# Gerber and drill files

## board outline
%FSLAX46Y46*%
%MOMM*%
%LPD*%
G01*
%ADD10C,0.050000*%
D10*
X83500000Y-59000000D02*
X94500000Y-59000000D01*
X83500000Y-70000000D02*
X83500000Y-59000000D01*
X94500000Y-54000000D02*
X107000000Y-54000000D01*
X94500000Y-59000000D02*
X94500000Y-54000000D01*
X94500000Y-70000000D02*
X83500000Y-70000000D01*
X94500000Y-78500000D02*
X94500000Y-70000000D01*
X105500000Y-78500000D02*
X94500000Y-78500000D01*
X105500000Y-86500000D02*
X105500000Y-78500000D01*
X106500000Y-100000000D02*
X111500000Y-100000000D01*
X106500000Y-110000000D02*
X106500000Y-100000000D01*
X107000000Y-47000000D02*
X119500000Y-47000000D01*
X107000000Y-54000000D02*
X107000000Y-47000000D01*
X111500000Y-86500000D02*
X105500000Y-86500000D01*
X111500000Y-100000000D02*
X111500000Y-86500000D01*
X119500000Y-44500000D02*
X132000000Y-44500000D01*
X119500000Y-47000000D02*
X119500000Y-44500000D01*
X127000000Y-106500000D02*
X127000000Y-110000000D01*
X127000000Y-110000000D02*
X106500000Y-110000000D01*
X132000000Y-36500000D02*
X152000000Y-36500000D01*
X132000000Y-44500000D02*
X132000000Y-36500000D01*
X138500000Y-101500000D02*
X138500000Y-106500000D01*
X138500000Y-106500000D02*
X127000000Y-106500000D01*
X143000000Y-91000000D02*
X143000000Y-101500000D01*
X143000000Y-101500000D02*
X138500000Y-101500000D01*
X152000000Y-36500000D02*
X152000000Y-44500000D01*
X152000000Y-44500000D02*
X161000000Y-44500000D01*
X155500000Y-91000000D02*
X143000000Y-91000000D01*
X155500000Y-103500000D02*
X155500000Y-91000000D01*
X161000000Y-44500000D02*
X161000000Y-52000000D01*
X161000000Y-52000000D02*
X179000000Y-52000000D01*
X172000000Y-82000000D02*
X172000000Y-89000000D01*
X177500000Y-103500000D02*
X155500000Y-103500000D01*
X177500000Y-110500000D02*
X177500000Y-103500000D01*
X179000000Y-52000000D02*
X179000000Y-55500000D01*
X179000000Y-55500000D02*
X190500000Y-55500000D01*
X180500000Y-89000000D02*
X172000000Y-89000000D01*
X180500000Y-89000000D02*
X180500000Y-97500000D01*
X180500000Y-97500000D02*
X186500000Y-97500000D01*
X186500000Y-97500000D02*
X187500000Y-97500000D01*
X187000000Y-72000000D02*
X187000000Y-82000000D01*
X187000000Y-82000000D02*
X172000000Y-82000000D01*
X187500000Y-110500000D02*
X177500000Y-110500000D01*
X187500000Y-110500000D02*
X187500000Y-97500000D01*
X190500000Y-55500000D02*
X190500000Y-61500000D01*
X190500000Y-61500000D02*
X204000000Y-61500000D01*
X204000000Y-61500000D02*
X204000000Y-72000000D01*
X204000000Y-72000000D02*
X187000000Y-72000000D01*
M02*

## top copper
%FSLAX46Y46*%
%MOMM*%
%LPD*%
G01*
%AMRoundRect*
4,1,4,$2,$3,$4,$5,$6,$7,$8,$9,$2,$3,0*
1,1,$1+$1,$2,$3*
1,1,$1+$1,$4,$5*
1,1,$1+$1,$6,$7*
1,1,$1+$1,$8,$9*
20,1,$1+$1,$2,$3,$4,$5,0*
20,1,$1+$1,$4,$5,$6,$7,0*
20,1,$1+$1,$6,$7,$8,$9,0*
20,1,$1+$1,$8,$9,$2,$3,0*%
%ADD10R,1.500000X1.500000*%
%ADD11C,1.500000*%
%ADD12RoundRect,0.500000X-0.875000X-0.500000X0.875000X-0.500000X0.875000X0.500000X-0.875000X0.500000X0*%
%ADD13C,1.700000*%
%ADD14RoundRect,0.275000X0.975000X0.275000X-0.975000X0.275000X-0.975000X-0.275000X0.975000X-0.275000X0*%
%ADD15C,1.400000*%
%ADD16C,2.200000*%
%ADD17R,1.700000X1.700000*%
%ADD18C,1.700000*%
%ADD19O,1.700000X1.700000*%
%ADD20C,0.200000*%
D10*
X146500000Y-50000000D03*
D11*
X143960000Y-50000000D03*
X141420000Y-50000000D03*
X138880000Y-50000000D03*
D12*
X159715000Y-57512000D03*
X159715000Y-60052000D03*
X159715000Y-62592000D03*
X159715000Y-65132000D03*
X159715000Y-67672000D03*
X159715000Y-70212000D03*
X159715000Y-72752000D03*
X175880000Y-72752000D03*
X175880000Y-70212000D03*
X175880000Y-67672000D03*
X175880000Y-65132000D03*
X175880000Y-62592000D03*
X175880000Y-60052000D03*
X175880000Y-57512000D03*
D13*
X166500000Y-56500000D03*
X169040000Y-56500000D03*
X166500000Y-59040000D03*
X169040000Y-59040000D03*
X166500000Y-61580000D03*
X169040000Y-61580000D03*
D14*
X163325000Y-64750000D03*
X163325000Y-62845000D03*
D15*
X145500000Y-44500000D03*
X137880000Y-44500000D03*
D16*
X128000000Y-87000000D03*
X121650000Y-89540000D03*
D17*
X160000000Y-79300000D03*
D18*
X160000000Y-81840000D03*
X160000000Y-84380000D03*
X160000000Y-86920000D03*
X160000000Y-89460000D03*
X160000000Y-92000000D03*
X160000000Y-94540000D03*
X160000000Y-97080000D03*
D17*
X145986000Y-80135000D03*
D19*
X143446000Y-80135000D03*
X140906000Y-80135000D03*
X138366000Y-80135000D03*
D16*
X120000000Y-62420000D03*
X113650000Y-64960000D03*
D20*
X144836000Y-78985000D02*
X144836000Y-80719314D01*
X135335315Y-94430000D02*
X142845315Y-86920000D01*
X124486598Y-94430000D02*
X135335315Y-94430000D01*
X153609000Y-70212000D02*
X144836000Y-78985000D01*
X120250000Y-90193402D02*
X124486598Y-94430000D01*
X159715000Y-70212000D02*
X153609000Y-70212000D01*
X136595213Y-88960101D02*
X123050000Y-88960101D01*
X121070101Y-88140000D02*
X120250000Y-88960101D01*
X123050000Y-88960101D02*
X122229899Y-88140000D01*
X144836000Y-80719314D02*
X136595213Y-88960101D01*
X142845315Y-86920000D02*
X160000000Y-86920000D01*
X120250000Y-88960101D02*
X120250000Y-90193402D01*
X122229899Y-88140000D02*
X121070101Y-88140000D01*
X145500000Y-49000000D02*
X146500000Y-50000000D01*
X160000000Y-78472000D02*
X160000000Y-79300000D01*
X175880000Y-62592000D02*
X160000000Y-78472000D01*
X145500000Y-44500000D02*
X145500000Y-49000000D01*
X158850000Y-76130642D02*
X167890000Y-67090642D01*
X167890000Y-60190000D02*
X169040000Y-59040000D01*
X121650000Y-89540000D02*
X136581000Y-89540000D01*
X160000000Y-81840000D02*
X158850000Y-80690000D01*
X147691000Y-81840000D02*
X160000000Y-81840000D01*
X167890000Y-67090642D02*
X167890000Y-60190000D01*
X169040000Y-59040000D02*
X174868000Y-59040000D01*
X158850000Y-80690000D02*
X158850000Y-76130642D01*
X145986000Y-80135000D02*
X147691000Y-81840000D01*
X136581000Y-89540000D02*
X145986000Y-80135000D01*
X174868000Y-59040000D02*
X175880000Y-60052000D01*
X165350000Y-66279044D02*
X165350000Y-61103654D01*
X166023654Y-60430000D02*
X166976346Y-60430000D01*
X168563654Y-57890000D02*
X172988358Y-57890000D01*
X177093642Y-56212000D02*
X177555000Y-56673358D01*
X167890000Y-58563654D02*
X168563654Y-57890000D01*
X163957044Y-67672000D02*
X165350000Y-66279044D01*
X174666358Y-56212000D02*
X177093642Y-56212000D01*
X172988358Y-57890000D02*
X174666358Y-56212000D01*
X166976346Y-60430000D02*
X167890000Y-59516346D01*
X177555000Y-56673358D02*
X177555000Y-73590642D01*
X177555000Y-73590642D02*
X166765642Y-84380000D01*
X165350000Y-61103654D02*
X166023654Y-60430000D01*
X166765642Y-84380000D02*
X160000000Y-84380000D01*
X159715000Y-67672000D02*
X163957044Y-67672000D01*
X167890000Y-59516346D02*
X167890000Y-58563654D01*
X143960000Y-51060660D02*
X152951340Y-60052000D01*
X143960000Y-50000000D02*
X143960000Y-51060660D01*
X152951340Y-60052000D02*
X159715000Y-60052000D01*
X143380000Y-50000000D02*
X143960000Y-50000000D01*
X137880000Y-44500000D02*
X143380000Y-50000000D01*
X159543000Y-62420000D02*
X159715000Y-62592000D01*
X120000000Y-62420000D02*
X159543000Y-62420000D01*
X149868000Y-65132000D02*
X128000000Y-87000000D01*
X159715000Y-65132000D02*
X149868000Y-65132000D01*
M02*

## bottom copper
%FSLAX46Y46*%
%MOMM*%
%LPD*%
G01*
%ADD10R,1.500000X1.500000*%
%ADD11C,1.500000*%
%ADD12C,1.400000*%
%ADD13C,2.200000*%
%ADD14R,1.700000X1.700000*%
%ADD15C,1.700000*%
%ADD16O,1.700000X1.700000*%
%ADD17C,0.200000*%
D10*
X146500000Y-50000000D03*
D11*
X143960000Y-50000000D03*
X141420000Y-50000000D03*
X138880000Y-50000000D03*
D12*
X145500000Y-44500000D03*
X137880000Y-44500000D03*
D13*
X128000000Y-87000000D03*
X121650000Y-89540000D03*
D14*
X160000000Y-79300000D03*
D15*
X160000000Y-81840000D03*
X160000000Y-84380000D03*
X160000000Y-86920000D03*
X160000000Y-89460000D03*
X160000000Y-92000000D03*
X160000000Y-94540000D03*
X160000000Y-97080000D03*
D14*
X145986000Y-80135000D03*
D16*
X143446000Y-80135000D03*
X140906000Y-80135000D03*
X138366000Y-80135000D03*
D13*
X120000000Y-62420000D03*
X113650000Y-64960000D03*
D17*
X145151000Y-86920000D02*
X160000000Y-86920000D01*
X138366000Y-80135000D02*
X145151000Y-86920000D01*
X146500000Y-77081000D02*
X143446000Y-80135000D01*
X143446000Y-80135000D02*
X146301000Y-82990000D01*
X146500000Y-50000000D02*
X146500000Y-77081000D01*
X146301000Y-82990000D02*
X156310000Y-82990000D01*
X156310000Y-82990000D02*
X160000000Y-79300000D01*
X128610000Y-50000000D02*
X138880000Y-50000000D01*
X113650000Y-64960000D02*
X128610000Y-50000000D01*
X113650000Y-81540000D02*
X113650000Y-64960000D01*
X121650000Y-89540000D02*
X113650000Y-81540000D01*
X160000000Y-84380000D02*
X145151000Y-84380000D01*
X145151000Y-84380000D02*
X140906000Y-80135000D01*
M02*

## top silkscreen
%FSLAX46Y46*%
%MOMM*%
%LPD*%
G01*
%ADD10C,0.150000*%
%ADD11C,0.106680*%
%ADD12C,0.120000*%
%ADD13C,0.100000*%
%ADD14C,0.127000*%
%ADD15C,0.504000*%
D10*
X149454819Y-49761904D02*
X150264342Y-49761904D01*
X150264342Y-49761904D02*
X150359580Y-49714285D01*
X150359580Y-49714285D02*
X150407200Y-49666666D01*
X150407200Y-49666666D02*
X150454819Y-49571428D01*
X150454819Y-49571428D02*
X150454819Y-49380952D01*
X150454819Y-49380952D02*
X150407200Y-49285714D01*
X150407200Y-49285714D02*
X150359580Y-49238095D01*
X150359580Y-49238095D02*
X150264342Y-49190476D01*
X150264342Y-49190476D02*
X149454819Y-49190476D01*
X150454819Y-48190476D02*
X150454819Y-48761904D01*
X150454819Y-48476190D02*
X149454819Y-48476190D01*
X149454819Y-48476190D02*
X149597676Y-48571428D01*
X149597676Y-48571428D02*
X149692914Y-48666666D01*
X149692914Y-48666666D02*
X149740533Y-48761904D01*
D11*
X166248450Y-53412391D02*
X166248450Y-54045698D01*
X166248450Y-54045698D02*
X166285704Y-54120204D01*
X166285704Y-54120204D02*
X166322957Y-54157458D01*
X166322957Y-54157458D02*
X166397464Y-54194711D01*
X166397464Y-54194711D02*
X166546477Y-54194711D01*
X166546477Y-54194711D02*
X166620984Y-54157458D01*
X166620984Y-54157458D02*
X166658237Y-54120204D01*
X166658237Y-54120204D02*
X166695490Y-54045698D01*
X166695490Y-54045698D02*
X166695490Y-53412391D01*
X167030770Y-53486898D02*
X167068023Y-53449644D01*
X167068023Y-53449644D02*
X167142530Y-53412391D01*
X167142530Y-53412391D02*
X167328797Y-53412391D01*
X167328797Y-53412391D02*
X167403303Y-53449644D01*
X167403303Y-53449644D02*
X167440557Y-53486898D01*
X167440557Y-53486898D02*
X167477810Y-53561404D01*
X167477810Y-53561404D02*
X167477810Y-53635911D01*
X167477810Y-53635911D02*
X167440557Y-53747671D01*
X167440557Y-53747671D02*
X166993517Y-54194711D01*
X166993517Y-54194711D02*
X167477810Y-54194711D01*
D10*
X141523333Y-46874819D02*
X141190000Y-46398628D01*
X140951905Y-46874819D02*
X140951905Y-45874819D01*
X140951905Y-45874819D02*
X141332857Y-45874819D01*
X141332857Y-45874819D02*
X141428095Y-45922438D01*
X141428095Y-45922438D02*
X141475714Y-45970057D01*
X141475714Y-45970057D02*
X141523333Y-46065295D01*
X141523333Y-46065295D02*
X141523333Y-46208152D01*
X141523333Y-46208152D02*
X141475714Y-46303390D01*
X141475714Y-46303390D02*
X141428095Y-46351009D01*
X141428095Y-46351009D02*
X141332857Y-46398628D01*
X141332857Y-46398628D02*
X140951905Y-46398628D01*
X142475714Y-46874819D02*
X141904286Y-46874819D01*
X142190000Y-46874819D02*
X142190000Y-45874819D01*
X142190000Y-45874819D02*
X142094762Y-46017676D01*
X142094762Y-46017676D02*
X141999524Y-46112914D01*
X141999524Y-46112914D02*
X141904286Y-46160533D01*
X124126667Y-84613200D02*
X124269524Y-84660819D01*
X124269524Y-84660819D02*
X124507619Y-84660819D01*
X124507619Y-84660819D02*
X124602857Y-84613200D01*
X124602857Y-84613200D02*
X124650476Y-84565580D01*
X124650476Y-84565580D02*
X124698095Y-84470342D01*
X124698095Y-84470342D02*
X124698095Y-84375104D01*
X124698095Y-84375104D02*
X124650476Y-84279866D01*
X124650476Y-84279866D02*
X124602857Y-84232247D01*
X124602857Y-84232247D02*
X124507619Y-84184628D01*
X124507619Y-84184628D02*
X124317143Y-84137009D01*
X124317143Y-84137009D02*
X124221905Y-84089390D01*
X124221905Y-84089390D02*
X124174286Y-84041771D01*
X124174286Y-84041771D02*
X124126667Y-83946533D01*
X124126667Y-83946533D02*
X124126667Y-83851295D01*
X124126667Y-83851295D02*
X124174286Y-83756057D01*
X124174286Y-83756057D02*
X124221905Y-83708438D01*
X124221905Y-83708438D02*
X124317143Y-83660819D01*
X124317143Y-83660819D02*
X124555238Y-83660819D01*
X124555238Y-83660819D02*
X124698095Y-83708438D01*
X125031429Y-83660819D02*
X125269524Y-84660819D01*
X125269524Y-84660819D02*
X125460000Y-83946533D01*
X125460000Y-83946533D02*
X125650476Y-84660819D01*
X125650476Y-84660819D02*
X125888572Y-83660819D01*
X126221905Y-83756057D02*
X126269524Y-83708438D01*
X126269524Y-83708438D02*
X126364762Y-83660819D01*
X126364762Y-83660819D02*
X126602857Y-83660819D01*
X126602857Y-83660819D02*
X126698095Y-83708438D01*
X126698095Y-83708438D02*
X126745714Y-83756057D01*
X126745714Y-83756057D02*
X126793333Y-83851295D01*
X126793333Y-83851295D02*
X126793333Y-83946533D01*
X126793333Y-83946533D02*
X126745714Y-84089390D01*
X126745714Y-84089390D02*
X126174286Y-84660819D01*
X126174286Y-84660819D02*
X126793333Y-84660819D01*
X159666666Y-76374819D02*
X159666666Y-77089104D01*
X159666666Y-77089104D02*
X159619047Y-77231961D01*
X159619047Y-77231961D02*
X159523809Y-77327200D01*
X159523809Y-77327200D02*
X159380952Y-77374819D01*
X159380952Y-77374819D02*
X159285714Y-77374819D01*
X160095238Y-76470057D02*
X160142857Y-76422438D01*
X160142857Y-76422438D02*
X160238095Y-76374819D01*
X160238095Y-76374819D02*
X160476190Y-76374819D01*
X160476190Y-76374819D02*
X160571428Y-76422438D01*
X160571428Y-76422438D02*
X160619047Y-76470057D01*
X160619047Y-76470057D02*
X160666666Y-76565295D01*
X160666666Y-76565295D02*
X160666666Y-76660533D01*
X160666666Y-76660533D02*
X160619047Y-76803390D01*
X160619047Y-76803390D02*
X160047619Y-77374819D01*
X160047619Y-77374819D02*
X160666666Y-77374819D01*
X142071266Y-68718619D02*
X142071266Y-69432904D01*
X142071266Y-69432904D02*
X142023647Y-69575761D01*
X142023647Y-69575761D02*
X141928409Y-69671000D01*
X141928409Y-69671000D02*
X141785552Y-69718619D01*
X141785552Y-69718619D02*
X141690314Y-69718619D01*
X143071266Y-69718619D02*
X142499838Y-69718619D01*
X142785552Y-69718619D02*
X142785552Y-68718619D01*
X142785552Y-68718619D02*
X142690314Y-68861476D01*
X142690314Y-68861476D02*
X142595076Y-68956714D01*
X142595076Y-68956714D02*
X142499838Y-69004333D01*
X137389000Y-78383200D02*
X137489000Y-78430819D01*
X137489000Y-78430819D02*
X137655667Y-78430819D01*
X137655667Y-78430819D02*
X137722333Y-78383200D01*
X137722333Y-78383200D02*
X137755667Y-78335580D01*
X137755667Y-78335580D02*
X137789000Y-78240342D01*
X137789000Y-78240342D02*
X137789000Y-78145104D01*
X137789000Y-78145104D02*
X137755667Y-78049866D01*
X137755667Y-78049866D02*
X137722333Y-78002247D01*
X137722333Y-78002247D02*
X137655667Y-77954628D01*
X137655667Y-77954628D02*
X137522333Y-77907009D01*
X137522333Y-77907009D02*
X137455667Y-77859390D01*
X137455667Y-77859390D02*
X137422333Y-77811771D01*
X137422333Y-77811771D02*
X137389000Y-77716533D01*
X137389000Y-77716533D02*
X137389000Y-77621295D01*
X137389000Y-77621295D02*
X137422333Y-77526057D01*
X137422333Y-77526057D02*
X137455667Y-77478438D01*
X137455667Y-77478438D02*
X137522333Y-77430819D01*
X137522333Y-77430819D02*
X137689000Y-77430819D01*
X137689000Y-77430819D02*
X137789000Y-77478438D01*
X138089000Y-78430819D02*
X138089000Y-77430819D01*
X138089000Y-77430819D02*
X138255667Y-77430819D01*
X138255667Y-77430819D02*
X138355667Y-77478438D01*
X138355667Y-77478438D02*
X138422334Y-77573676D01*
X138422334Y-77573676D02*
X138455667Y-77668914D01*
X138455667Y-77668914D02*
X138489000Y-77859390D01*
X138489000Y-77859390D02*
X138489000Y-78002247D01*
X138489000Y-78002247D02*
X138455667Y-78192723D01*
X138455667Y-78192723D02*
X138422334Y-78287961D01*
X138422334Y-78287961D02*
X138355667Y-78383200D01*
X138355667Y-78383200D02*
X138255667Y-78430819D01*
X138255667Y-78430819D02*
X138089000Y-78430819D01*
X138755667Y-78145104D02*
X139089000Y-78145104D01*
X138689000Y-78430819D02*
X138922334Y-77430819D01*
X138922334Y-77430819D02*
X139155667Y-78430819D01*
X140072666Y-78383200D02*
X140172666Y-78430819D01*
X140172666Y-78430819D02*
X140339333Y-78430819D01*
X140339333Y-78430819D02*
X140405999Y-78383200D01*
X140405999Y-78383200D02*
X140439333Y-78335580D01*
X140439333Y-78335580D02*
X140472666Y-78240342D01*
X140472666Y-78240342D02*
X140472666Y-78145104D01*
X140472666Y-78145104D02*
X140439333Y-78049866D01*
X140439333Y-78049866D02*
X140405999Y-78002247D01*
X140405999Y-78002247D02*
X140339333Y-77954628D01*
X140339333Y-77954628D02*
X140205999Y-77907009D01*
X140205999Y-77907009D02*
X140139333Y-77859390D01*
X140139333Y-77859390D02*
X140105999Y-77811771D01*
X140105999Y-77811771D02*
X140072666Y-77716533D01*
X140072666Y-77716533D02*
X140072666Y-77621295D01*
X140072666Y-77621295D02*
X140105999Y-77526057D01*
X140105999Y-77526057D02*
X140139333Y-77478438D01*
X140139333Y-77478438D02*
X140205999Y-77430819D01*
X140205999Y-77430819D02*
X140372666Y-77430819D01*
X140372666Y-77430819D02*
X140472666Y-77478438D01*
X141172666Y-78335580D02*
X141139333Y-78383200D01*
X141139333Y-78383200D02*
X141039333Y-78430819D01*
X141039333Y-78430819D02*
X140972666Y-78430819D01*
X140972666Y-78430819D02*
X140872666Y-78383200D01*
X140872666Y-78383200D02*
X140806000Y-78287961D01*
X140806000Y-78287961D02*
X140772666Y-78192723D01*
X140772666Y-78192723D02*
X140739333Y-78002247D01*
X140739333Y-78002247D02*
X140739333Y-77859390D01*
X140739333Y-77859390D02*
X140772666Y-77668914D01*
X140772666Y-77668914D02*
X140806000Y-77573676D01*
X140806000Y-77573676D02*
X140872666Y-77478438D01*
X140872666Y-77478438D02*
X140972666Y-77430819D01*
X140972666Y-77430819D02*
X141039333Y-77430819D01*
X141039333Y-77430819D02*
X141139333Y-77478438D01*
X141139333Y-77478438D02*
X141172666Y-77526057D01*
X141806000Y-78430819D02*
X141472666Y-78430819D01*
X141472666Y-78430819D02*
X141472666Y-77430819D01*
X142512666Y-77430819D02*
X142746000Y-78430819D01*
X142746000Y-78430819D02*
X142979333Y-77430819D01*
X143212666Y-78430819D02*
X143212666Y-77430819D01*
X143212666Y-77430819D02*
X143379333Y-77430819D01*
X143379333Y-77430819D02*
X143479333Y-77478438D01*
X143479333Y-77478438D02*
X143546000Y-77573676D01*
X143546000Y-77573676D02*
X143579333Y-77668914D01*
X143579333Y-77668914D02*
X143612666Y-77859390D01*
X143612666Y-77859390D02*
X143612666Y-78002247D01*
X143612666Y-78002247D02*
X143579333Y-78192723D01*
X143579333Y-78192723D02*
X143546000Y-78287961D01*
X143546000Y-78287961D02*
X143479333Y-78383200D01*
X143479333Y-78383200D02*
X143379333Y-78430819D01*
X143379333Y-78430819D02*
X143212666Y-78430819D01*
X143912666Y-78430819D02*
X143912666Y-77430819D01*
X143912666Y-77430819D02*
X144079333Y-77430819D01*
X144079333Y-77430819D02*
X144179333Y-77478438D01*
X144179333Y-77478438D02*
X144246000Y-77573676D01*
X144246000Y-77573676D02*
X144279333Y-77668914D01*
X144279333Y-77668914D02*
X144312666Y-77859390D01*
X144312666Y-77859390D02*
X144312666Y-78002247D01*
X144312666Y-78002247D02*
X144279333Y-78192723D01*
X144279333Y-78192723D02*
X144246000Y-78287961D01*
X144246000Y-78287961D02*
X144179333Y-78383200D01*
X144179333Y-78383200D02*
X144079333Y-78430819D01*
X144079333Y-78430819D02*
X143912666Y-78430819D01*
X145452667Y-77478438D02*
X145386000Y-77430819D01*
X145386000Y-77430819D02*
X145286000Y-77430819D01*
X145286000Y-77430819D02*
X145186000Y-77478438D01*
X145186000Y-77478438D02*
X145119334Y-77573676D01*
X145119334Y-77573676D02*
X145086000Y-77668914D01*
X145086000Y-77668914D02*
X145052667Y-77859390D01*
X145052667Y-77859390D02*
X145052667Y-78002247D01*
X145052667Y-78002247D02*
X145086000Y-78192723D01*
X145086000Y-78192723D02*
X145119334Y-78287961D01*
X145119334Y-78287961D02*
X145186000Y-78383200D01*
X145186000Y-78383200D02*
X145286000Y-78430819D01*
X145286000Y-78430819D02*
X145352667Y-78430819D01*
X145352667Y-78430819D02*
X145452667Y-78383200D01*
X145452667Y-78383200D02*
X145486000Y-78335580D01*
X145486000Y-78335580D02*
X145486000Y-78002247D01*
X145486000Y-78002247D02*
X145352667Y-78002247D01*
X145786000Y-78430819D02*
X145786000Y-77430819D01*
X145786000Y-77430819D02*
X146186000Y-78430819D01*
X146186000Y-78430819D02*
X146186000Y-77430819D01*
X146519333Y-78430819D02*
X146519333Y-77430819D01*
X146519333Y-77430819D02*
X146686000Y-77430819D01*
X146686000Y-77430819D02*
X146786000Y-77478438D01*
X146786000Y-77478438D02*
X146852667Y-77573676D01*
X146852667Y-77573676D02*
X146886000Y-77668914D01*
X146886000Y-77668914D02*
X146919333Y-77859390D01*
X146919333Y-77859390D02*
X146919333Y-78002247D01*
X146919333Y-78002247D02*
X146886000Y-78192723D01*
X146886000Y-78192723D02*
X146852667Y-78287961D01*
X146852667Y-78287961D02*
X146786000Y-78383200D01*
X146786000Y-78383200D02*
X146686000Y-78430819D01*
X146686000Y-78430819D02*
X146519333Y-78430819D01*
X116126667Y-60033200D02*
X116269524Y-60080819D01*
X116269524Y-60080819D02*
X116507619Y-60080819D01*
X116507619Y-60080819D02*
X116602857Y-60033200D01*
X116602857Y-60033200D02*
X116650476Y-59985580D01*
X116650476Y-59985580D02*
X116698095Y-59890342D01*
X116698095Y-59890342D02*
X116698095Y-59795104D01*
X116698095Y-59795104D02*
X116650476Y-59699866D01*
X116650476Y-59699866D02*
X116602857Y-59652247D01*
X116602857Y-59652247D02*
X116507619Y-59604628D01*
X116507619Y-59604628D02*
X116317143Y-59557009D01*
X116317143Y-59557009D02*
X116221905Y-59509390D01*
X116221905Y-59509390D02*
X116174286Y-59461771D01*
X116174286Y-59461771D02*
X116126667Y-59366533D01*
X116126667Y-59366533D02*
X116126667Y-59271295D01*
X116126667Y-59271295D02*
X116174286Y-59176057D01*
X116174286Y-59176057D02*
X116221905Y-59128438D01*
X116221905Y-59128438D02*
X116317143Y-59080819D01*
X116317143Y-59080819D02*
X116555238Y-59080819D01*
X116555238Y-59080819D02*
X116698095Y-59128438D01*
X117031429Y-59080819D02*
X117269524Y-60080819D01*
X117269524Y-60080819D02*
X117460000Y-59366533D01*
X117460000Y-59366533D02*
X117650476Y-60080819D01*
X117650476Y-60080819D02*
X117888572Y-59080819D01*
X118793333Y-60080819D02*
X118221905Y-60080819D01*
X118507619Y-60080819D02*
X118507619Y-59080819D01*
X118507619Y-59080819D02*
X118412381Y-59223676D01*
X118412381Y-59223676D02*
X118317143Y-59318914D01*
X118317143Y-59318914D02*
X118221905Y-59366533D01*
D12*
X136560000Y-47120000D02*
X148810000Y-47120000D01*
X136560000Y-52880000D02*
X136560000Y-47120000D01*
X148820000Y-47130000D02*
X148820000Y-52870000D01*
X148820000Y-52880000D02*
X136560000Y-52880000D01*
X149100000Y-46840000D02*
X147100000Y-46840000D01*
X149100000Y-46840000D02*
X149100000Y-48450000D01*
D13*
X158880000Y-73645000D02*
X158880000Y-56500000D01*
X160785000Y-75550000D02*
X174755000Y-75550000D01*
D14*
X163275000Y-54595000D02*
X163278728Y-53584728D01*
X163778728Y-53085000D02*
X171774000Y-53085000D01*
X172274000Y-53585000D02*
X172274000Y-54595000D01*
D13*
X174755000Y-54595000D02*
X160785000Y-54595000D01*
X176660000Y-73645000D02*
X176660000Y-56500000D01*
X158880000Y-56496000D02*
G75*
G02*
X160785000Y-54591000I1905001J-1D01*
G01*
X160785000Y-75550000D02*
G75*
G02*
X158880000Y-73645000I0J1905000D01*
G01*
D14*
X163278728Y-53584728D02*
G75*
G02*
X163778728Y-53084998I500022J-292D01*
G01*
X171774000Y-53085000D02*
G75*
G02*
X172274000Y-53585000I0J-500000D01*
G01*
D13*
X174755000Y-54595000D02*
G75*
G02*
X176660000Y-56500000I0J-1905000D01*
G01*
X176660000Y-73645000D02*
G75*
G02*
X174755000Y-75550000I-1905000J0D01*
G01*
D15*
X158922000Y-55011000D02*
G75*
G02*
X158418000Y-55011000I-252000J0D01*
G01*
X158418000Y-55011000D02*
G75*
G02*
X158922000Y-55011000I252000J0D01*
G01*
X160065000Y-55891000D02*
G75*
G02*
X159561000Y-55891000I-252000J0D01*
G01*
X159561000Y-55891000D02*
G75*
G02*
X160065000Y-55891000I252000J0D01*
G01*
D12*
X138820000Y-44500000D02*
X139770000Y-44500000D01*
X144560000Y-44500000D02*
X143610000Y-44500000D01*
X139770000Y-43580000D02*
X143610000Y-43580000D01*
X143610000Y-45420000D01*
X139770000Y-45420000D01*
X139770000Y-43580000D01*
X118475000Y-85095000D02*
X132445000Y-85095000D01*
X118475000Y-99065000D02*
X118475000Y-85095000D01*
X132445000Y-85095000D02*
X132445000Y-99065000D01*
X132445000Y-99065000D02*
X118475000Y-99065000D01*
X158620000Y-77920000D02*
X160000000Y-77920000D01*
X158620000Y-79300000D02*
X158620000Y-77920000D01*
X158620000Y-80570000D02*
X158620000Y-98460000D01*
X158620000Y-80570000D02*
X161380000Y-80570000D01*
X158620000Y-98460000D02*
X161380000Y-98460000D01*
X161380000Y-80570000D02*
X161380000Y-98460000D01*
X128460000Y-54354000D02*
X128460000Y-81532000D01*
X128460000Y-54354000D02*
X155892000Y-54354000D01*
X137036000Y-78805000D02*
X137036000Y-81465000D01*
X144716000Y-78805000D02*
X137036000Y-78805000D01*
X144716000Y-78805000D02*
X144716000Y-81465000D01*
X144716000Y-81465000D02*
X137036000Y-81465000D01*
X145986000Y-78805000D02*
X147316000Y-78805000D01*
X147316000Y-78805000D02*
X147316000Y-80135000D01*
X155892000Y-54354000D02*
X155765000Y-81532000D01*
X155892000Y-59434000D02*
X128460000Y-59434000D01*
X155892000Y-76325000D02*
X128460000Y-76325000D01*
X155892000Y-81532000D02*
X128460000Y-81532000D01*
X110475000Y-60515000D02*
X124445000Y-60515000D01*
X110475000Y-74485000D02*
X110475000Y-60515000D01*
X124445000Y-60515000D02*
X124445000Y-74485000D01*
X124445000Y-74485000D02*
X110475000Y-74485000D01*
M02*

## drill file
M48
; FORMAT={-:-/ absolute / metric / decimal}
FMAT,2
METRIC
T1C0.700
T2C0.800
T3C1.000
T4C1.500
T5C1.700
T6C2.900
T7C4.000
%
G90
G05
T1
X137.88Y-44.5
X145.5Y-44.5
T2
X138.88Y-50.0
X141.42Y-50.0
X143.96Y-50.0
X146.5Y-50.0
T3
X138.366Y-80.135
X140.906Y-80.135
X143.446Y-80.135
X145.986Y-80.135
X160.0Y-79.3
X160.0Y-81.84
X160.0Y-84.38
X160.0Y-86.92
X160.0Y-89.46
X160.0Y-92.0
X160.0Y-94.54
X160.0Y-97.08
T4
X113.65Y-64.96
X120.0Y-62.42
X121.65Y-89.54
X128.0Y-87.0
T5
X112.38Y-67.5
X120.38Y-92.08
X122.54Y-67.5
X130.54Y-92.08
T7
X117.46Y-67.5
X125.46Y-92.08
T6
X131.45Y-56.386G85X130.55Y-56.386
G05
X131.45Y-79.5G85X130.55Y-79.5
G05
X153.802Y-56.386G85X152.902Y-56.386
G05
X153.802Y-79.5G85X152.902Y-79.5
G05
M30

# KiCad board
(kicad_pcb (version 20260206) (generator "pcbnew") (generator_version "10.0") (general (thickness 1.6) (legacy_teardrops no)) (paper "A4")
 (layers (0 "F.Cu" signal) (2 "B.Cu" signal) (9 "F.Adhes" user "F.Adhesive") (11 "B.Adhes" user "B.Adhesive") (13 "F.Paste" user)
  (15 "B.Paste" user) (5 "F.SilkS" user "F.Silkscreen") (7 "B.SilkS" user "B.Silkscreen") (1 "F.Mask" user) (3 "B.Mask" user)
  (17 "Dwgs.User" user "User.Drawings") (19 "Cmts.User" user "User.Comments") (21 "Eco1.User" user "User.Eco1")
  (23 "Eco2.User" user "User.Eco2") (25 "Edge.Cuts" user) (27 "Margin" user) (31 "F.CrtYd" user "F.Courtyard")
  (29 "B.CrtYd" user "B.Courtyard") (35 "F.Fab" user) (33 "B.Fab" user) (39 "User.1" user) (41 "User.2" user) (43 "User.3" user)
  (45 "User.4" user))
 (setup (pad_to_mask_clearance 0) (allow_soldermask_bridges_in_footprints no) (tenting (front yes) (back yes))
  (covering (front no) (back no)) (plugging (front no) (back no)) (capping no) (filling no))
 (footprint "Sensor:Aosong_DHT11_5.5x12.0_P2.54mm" (layer "F.Cu") (at 146.5 50 -90)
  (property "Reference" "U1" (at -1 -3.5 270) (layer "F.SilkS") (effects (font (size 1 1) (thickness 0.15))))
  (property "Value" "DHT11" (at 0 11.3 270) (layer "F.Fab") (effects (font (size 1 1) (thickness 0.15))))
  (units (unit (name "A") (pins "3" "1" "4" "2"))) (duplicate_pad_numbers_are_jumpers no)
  (fp_line (start -2.88 9.94) (end -2.88 -2.31) (stroke (width 0.12) (type solid)) (layer "F.SilkS"))
  (fp_line (start 2.88 9.94) (end -2.88 9.94) (stroke (width 0.12) (type solid)) (layer "F.SilkS"))
  (fp_line (start -2.87 -2.32) (end 2.87 -2.32) (stroke (width 0.12) (type solid)) (layer "F.SilkS"))
  (fp_line (start 2.88 -2.32) (end 2.88 9.94) (stroke (width 0.12) (type solid)) (layer "F.SilkS"))
  (fp_line (start -3.16 -2.6) (end -3.16 -0.6) (stroke (width 0.12) (type solid)) (layer "F.SilkS"))
  (fp_line (start -3.16 -2.6) (end -1.55 -2.6) (stroke (width 0.12) (type solid)) (layer "F.SilkS"))
  (pad "1" thru_hole rect (at 0 0 270) (size 1.5 1.5) (drill 0.8) (layers "*.Cu" "*.Mask") (remove_unused_layers no) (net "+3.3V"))
  (pad "2" thru_hole circle (at 0 2.54 270) (size 1.5 1.5) (drill 0.8) (layers "*.Cu" "*.Mask") (remove_unused_layers no)
   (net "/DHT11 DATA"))
  (pad "3" thru_hole circle (at 0 5.08 270) (size 1.5 1.5) (drill 0.8) (layers "*.Cu" "*.Mask") (remove_unused_layers no)
   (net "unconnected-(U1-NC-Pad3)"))
  (pad "4" thru_hole circle (at 0 7.62 270) (size 1.5 1.5) (drill 0.8) (layers "*.Cu" "*.Mask") (remove_unused_layers no) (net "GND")))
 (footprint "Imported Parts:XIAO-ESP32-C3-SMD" (layer "F.Cu") (at 158.88 75.632)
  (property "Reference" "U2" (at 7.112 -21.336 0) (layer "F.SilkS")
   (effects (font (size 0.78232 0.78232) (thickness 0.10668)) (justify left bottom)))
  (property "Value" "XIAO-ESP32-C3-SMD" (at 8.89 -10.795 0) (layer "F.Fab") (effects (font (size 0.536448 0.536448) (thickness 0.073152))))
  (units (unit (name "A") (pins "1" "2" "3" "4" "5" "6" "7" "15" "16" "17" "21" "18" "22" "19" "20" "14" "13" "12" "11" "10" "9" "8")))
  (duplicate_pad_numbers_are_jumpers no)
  (fp_line (start 0 -1.987) (end 0 -19.132) (stroke (width 0.1) (type solid)) (layer "F.SilkS"))
  (fp_line (start 1.905 -0.082) (end 15.875 -0.082) (stroke (width 0.1) (type solid)) (layer "F.SilkS"))
  (fp_line (start 4.395 -21.037) (end 4.398728 -22.047272) (stroke (width 0.127) (type solid)) (layer "F.SilkS"))
  (fp_line (start 4.898728 -22.547) (end 12.894 -22.547) (stroke (width 0.127) (type solid)) (layer "F.SilkS"))
  (fp_line (start 13.394 -22.047) (end 13.394 -21.037) (stroke (width 0.127) (type solid)) (layer "F.SilkS"))
  (fp_line (start 15.875 -21.037) (end 1.905 -21.037) (stroke (width 0.1) (type solid)) (layer "F.SilkS"))
  (fp_line (start 17.78 -1.987) (end 17.78 -19.132) (stroke (width 0.1) (type solid)) (layer "F.SilkS"))
  (fp_arc (start 0 -19.136) (mid 0.557962 -20.483038) (end 1.905 -21.041) (stroke (width 0.1) (type solid)) (layer "F.SilkS"))
  (fp_arc (start 1.905 -0.082) (mid 0.557962 -0.639962) (end 0 -1.987) (stroke (width 0.1) (type solid)) (layer "F.SilkS"))
  (fp_arc (start 4.398728 -22.047272) (mid 4.545272 -22.40064) (end 4.898728 -22.547) (stroke (width 0.127) (type default))
   (layer "F.SilkS"))
  (fp_arc (start 12.894 -22.547) (mid 13.247553 -22.400553) (end 13.394 -22.047) (stroke (width 0.127) (type default)) (layer "F.SilkS"))
  (fp_arc (start 15.875 -21.037) (mid 17.222038 -20.479038) (end 17.78 -19.132) (stroke (width 0.1) (type solid)) (layer "F.SilkS"))
  (fp_arc (start 17.78 -1.987) (mid 17.222038 -0.639962) (end 15.875 -0.082) (stroke (width 0.1) (type solid)) (layer "F.SilkS"))
  (fp_circle (center -0.21 -20.621) (end -0.21 -20.875) (stroke (width 0.5) (type solid)) (fill yes) (layer "F.SilkS"))
  (fp_circle (center 0.933 -19.741) (end 0.933 -19.995) (stroke (width 0.5) (type solid)) (fill yes) (layer "F.SilkS"))
  (pad "1" smd roundrect (at 0.835 -18.12) (size 2.75 2) (layers "F.Cu" "F.Mask" "F.Paste") (roundrect_rratio 0.25)
   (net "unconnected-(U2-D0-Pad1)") (solder_mask_margin 0.0508) (thermal_bridge_angle 45))
  (pad "2" smd roundrect (at 0.835 -15.58) (size 2.75 2) (layers "F.Cu" "F.Mask" "F.Paste") (roundrect_rratio 0.25) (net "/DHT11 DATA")
   (solder_mask_margin 0.0508) (thermal_bridge_angle 45))
  (pad "3" smd roundrect (at 0.835 -13.04) (size 2.75 2) (layers "F.Cu" "F.Mask" "F.Paste") (roundrect_rratio 0.25) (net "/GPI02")
   (solder_mask_margin 0.0508) (thermal_bridge_angle 45))
  (pad "4" smd roundrect (at 0.835 -10.5) (size 2.75 2) (layers "F.Cu" "F.Mask" "F.Paste") (roundrect_rratio 0.25) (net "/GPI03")
   (solder_mask_margin 0.0508) (thermal_bridge_angle 45))
  (pad "5" smd roundrect (at 0.835 -7.96) (size 2.75 2) (layers "F.Cu" "F.Mask" "F.Paste") (roundrect_rratio 0.25) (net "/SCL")
   (solder_mask_margin 0.0508) (thermal_bridge_angle 45))
  (pad "6" smd roundrect (at 0.835 -5.42) (size 2.75 2) (layers "F.Cu" "F.Mask" "F.Paste") (roundrect_rratio 0.25) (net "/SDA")
   (solder_mask_margin 0.0508) (thermal_bridge_angle 45))
  (pad "7" smd roundrect (at 0.835 -2.88) (size 2.75 2) (layers "F.Cu" "F.Mask" "F.Paste") (roundrect_rratio 0.25)
   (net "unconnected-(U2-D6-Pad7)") (solder_mask_margin 0.0508) (thermal_bridge_angle 45))
  (pad "8" smd roundrect (at 17 -2.88) (size 2.75 2) (layers "F.Cu" "F.Mask" "F.Paste") (roundrect_rratio 0.25)
   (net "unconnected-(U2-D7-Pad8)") (solder_mask_margin 0.0508) (thermal_bridge_angle 45))
  (pad "9" smd roundrect (at 17 -5.42) (size 2.75 2) (layers "F.Cu" "F.Mask" "F.Paste") (roundrect_rratio 0.25)
   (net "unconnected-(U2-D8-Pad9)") (solder_mask_margin 0.0508) (thermal_bridge_angle 45))
  (pad "10" smd roundrect (at 17 -7.96) (size 2.75 2) (layers "F.Cu" "F.Mask" "F.Paste") (roundrect_rratio 0.25)
   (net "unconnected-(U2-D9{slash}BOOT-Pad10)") (solder_mask_margin 0.0508) (thermal_bridge_angle 45))
  (pad "11" smd roundrect (at 17 -10.5) (size 2.75 2) (layers "F.Cu" "F.Mask" "F.Paste") (roundrect_rratio 0.25)
   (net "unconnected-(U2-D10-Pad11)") (solder_mask_margin 0.0508) (thermal_bridge_angle 45))
  (pad "12" smd roundrect (at 17 -13.04) (size 2.75 2) (layers "F.Cu" "F.Mask" "F.Paste") (roundrect_rratio 0.25) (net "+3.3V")
   (solder_mask_margin 0.0508) (thermal_bridge_angle 45))
  (pad "13" smd roundrect (at 17 -15.58) (size 2.75 2) (layers "F.Cu" "F.Mask" "F.Paste") (roundrect_rratio 0.25) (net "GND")
   (solder_mask_margin 0.0508) (thermal_bridge_angle 45))
  (pad "14" smd roundrect (at 17 -18.12) (size 2.75 2) (layers "F.Cu" "F.Mask" "F.Paste") (roundrect_rratio 0.25) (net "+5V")
   (solder_mask_margin 0.0508) (thermal_bridge_angle 45))
  (pad "15" smd circle (at 7.62 -19.132) (size 1.7 1.7) (layers "F.Cu" "F.Mask" "F.Paste") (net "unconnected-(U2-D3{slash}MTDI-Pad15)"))
  (pad "16" smd circle (at 10.16 -19.132) (size 1.7 1.7) (layers "F.Cu" "F.Mask" "F.Paste") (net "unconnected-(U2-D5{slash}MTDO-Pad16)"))
  (pad "17" smd circle (at 7.62 -16.592) (size 1.7 1.7) (layers "F.Cu" "F.Mask" "F.Paste") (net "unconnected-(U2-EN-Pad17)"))
  (pad "18" smd circle (at 10.16 -16.592) (size 1.7 1.7) (layers "F.Cu" "F.Mask" "F.Paste") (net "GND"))
  (pad "19" smd circle (at 7.62 -14.052) (size 1.7 1.7) (layers "F.Cu" "F.Mask" "F.Paste") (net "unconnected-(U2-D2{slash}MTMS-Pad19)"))
  (pad "20" smd circle (at 10.16 -14.052) (size 1.7 1.7) (layers "F.Cu" "F.Mask" "F.Paste") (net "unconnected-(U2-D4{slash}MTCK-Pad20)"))
  (pad "21" smd roundrect (at 4.445 -10.882 180) (size 2.5 1.1) (layers "F.Cu" "F.Mask" "F.Paste") (roundrect_rratio 0.25)
   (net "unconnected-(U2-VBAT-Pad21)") (thermal_bridge_angle 45))
  (pad "22" smd roundrect (at 4.445 -12.787 180) (size 2.5 1.1) (layers "F.Cu" "F.Mask" "F.Paste") (roundrect_rratio 0.25)
   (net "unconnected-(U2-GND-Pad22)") (thermal_bridge_angle 45)))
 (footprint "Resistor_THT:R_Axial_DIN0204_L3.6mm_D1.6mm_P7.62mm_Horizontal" (layer "F.Cu") (at 145.5 44.5 180)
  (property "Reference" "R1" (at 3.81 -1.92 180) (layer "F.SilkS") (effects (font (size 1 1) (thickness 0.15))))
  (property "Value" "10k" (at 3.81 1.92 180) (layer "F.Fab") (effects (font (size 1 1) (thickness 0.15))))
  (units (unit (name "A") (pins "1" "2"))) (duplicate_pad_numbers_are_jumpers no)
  (fp_line (start 6.68 0) (end 5.73 0) (stroke (width 0.12) (type solid)) (layer "F.SilkS"))
  (fp_line (start 0.94 0) (end 1.89 0) (stroke (width 0.12) (type solid)) (layer "F.SilkS"))
  (fp_rect (start 1.89 -0.92) (end 5.73 0.92) (stroke (width 0.12) (type solid)) (fill no) (layer "F.SilkS"))
  (pad "1" thru_hole circle (at 0 0 180) (size 1.4 1.4) (drill 0.7) (layers "*.Cu" "*.Mask") (remove_unused_layers no) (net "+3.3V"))
  (pad "2" thru_hole circle (at 7.62 0 180) (size 1.4 1.4) (drill 0.7) (layers "*.Cu" "*.Mask") (remove_unused_layers no)
   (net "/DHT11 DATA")))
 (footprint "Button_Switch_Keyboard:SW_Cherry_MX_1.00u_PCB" (layer "F.Cu") (at 128 87)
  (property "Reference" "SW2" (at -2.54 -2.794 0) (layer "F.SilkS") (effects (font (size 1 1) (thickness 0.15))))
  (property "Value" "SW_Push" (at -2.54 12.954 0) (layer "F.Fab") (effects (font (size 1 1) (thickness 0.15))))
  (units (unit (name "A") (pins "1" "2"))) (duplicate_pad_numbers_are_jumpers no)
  (fp_line (start -9.525 -1.905) (end 4.445 -1.905) (stroke (width 0.12) (type solid)) (layer "F.SilkS"))
  (fp_line (start -9.525 12.065) (end -9.525 -1.905) (stroke (width 0.12) (type solid)) (layer "F.SilkS"))
  (fp_line (start 4.445 -1.905) (end 4.445 12.065) (stroke (width 0.12) (type solid)) (layer "F.SilkS"))
  (fp_line (start 4.445 12.065) (end -9.525 12.065) (stroke (width 0.12) (type solid)) (layer "F.SilkS"))
  (pad "" np_thru_hole circle (at -7.62 5.08) (size 1.7 1.7) (drill 1.7) (layers "*.Cu" "*.Mask"))
  (pad "" np_thru_hole circle (at -2.54 5.08) (size 4 4) (drill 4) (layers "*.Cu" "*.Mask"))
  (pad "" np_thru_hole circle (at 2.54 5.08) (size 1.7 1.7) (drill 1.7) (layers "*.Cu" "*.Mask"))
  (pad "1" thru_hole circle (at 0 0) (size 2.2 2.2) (drill 1.5) (layers "*.Cu" "*.Mask") (remove_unused_layers no) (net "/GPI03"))
  (pad "2" thru_hole circle (at -6.35 2.54) (size 2.2 2.2) (drill 1.5) (layers "*.Cu" "*.Mask") (remove_unused_layers no) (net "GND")))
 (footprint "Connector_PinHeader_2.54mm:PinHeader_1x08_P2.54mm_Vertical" (layer "F.Cu") (at 160 79.3)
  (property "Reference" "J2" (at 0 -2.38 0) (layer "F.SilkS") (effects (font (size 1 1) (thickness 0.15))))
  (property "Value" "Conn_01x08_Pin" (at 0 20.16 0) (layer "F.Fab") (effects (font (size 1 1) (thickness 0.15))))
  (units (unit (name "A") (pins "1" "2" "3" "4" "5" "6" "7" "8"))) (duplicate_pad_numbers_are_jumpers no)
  (fp_line (start -1.38 -1.38) (end 0 -1.38) (stroke (width 0.12) (type solid)) (layer "F.SilkS"))
  (fp_line (start -1.38 0) (end -1.38 -1.38) (stroke (width 0.12) (type solid)) (layer "F.SilkS"))
  (fp_line (start -1.38 1.27) (end -1.38 19.16) (stroke (width 0.12) (type solid)) (layer "F.SilkS"))
  (fp_line (start -1.38 1.27) (end 1.38 1.27) (stroke (width 0.12) (type solid)) (layer "F.SilkS"))
  (fp_line (start -1.38 19.16) (end 1.38 19.16) (stroke (width 0.12) (type solid)) (layer "F.SilkS"))
  (fp_line (start 1.38 1.27) (end 1.38 19.16) (stroke (width 0.12) (type solid)) (layer "F.SilkS"))
  (pad "1" thru_hole rect (at 0 0) (size 1.7 1.7) (drill 1) (layers "*.Cu" "*.Mask") (remove_unused_layers no) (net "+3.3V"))
  (pad "2" thru_hole circle (at 0 2.54) (size 1.7 1.7) (drill 1) (layers "*.Cu" "*.Mask") (remove_unused_layers no) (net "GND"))
  (pad "3" thru_hole circle (at 0 5.08) (size 1.7 1.7) (drill 1) (layers "*.Cu" "*.Mask") (remove_unused_layers no) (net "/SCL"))
  (pad "4" thru_hole circle (at 0 7.62) (size 1.7 1.7) (drill 1) (layers "*.Cu" "*.Mask") (remove_unused_layers no) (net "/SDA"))
  (pad "5" thru_hole circle (at 0 10.16) (size 1.7 1.7) (drill 1) (layers "*.Cu" "*.Mask") (remove_unused_layers no)
   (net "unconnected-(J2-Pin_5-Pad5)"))
  (pad "6" thru_hole circle (at 0 12.7) (size 1.7 1.7) (drill 1) (layers "*.Cu" "*.Mask") (remove_unused_layers no)
   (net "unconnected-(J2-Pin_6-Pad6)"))
  (pad "7" thru_hole circle (at 0 15.24) (size 1.7 1.7) (drill 1) (layers "*.Cu" "*.Mask") (remove_unused_layers no)
   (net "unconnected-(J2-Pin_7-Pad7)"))
  (pad "8" thru_hole circle (at 0 17.78) (size 1.7 1.7) (drill 1) (layers "*.Cu" "*.Mask") (remove_unused_layers no)
   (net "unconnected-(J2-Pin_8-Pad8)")))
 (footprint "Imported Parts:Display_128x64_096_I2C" (layer "F.Cu") (at 142.176 80.135 180)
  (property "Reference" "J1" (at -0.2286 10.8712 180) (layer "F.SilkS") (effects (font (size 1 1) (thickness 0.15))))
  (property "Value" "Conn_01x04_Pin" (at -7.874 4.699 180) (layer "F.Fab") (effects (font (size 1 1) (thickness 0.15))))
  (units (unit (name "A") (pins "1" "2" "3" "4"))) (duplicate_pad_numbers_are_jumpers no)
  (fp_line (start 13.716 25.781) (end 13.716 -1.397) (stroke (width 0.12) (type solid)) (layer "F.SilkS"))
  (fp_line (start 13.716 25.781) (end -13.716 25.781) (stroke (width 0.12) (type solid)) (layer "F.SilkS"))
  (fp_line (start 5.14 1.33) (end 5.14 -1.33) (stroke (width 0.12) (type solid)) (layer "F.SilkS"))
  (fp_line (start -2.54 1.33) (end 5.14 1.33) (stroke (width 0.12) (type solid)) (layer "F.SilkS"))
  (fp_line (start -2.54 1.33) (end -2.54 -1.33) (stroke (width 0.12) (type solid)) (layer "F.SilkS"))
  (fp_line (start -2.54 -1.33) (end 5.14 -1.33) (stroke (width 0.12) (type solid)) (layer "F.SilkS"))
  (fp_line (start -3.81 1.33) (end -5.14 1.33) (stroke (width 0.12) (type solid)) (layer "F.SilkS"))
  (fp_line (start -5.14 1.33) (end -5.14 0) (stroke (width 0.12) (type solid)) (layer "F.SilkS"))
  (fp_line (start -13.716 25.781) (end -13.589 -1.397) (stroke (width 0.12) (type solid)) (layer "F.SilkS"))
  (fp_line (start -13.716 20.701) (end 13.716 20.701) (stroke (width 0.12) (type solid)) (layer "F.SilkS"))
  (fp_line (start -13.716 3.81) (end 13.716 3.81) (stroke (width 0.12) (type solid)) (layer "F.SilkS"))
  (fp_line (start -13.716 -1.397) (end 13.716 -1.397) (stroke (width 0.12) (type solid)) (layer "F.SilkS"))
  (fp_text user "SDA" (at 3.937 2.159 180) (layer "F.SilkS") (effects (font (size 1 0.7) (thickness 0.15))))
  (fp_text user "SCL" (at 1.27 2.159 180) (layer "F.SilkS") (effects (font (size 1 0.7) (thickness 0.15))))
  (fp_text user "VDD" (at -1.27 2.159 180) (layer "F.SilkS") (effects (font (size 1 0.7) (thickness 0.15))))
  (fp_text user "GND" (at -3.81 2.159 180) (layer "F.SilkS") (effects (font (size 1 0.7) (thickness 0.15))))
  (pad "" np_thru_hole oval (at -11.176 0.635 180) (size 3.8 2.9) (drill oval 3.8 2.9) (layers "*.Cu" "*.Mask"))
  (pad "" np_thru_hole oval (at -11.176 23.749 180) (size 3.8 2.9) (drill oval 3.8 2.9) (layers "*.Cu" "*.Mask"))
  (pad "" np_thru_hole oval (at 11.176 0.635 180) (size 3.8 2.9) (drill oval 3.8 2.9) (layers "*.Cu" "*.Mask"))
  (pad "" np_thru_hole oval (at 11.176 23.749 180) (size 3.8 2.9) (drill oval 3.8 2.9) (layers "*.Cu" "*.Mask"))
  (pad "1" thru_hole rect (at -3.81 0 270) (size 1.7 1.7) (drill 1) (layers "*.Cu" "*.Mask") (remove_unused_layers no) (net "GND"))
  (pad "2" thru_hole oval (at -1.27 0 270) (size 1.7 1.7) (drill 1) (layers "*.Cu" "*.Mask") (remove_unused_layers no) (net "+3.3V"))
  (pad "3" thru_hole oval (at 1.27 0 270) (size 1.7 1.7) (drill 1) (layers "*.Cu" "*.Mask") (remove_unused_layers no) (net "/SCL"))
  (pad "4" thru_hole oval (at 3.81 0 270) (size 1.7 1.7) (drill 1) (layers "*.Cu" "*.Mask") (remove_unused_layers no) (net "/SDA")))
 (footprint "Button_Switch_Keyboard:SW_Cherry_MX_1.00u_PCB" (layer "F.Cu") (at 120 62.42)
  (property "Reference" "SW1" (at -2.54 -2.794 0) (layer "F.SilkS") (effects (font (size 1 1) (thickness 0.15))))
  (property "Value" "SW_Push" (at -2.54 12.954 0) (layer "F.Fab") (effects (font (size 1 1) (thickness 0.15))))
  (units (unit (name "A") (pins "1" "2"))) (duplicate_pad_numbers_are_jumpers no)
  (fp_line (start -9.525 -1.905) (end 4.445 -1.905) (stroke (width 0.12) (type solid)) (layer "F.SilkS"))
  (fp_line (start -9.525 12.065) (end -9.525 -1.905) (stroke (width 0.12) (type solid)) (layer "F.SilkS"))
  (fp_line (start 4.445 -1.905) (end 4.445 12.065) (stroke (width 0.12) (type solid)) (layer "F.SilkS"))
  (fp_line (start 4.445 12.065) (end -9.525 12.065) (stroke (width 0.12) (type solid)) (layer "F.SilkS"))
  (pad "" np_thru_hole circle (at -7.62 5.08) (size 1.7 1.7) (drill 1.7) (layers "*.Cu" "*.Mask"))
  (pad "" np_thru_hole circle (at -2.54 5.08) (size 4 4) (drill 4) (layers "*.Cu" "*.Mask"))
  (pad "" np_thru_hole circle (at 2.54 5.08) (size 1.7 1.7) (drill 1.7) (layers "*.Cu" "*.Mask"))
  (pad "1" thru_hole circle (at 0 0) (size 2.2 2.2) (drill 1.5) (layers "*.Cu" "*.Mask") (remove_unused_layers no) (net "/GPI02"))
  (pad "2" thru_hole circle (at -6.35 2.54) (size 2.2 2.2) (drill 1.5) (layers "*.Cu" "*.Mask") (remove_unused_layers no) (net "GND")))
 (gr_line (start 83.5 59) (end 94.5 59) (stroke (width 0.05) (type default)) (layer "Edge.Cuts"))
 (gr_line (start 83.5 70) (end 83.5 59) (stroke (width 0.05) (type default)) (layer "Edge.Cuts"))
 (gr_line (start 94.5 54) (end 107 54) (stroke (width 0.05) (type default)) (layer "Edge.Cuts"))
 (gr_line (start 94.5 59) (end 94.5 54) (stroke (width 0.05) (type default)) (layer "Edge.Cuts"))
 (gr_line (start 94.5 70) (end 83.5 70) (stroke (width 0.05) (type default)) (layer "Edge.Cuts"))
 (gr_line (start 94.5 78.5) (end 94.5 70) (stroke (width 0.05) (type default)) (layer "Edge.Cuts"))
 (gr_line (start 105.5 78.5) (end 94.5 78.5) (stroke (width 0.05) (type default)) (layer "Edge.Cuts"))
 (gr_line (start 105.5 86.5) (end 105.5 78.5) (stroke (width 0.05) (type default)) (layer "Edge.Cuts"))
 (gr_line (start 106.5 100) (end 111.5 100) (stroke (width 0.05) (type default)) (layer "Edge.Cuts"))
 (gr_line (start 106.5 110) (end 106.5 100) (stroke (width 0.05) (type default)) (layer "Edge.Cuts"))
 (gr_line (start 107 47) (end 119.5 47) (stroke (width 0.05) (type default)) (layer "Edge.Cuts"))
 (gr_line (start 107 54) (end 107 47) (stroke (width 0.05) (type default)) (layer "Edge.Cuts"))
 (gr_line (start 111.5 86.5) (end 105.5 86.5) (stroke (width 0.05) (type default)) (layer "Edge.Cuts"))
 (gr_line (start 111.5 100) (end 111.5 86.5) (stroke (width 0.05) (type default)) (layer "Edge.Cuts"))
 (gr_line (start 119.5 44.5) (end 132 44.5) (stroke (width 0.05) (type default)) (layer "Edge.Cuts"))
 (gr_line (start 119.5 47) (end 119.5 44.5) (stroke (width 0.05) (type default)) (layer "Edge.Cuts"))
 (gr_line (start 127 106.5) (end 127 110) (stroke (width 0.05) (type default)) (layer "Edge.Cuts"))
 (gr_line (start 127 110) (end 106.5 110) (stroke (width 0.05) (type default)) (layer "Edge.Cuts"))
 (gr_line (start 132 36.5) (end 152 36.5) (stroke (width 0.05) (type default)) (layer "Edge.Cuts"))
 (gr_line (start 132 44.5) (end 132 36.5) (stroke (width 0.05) (type default)) (layer "Edge.Cuts"))
 (gr_line (start 138.5 101.5) (end 138.5 106.5) (stroke (width 0.05) (type default)) (layer "Edge.Cuts"))
 (gr_line (start 138.5 106.5) (end 127 106.5) (stroke (width 0.05) (type default)) (layer "Edge.Cuts"))
 (gr_line (start 143 91) (end 143 101.5) (stroke (width 0.05) (type default)) (layer "Edge.Cuts"))
 (gr_line (start 143 101.5) (end 138.5 101.5) (stroke (width 0.05) (type default)) (layer "Edge.Cuts"))
 (gr_line (start 152 36.5) (end 152 44.5) (stroke (width 0.05) (type default)) (layer "Edge.Cuts"))
 (gr_line (start 152 44.5) (end 161 44.5) (stroke (width 0.05) (type default)) (layer "Edge.Cuts"))
 (gr_line (start 155.5 91) (end 143 91) (stroke (width 0.05) (type default)) (layer "Edge.Cuts"))
 (gr_line (start 155.5 103.5) (end 155.5 91) (stroke (width 0.05) (type default)) (layer "Edge.Cuts"))
 (gr_line (start 161 44.5) (end 161 52) (stroke (width 0.05) (type default)) (layer "Edge.Cuts"))
 (gr_line (start 161 52) (end 179 52) (stroke (width 0.05) (type default)) (layer "Edge.Cuts"))
 (gr_line (start 172 82) (end 172 89) (stroke (width 0.05) (type default)) (layer "Edge.Cuts"))
 (gr_line (start 177.5 103.5) (end 155.5 103.5) (stroke (width 0.05) (type default)) (layer "Edge.Cuts"))
 (gr_line (start 177.5 110.5) (end 177.5 103.5) (stroke (width 0.05) (type default)) (layer "Edge.Cuts"))
 (gr_line (start 179 52) (end 179 55.5) (stroke (width 0.05) (type default)) (layer "Edge.Cuts"))
 (gr_line (start 179 55.5) (end 190.5 55.5) (stroke (width 0.05) (type default)) (layer "Edge.Cuts"))
 (gr_line (start 180.5 89) (end 172 89) (stroke (width 0.05) (type default)) (layer "Edge.Cuts"))
 (gr_line (start 180.5 89) (end 180.5 97.5) (stroke (width 0.05) (type default)) (layer "Edge.Cuts"))
 (gr_line (start 180.5 97.5) (end 186.5 97.5) (stroke (width 0.05) (type default)) (layer "Edge.Cuts"))
 (gr_line (start 186.5 97.5) (end 187.5 97.5) (stroke (width 0.05) (type default)) (layer "Edge.Cuts"))
 (gr_line (start 187 72) (end 187 82) (stroke (width 0.05) (type default)) (layer "Edge.Cuts"))
 (gr_line (start 187 82) (end 172 82) (stroke (width 0.05) (type default)) (layer "Edge.Cuts"))
 (gr_line (start 187.5 110.5) (end 177.5 110.5) (stroke (width 0.05) (type default)) (layer "Edge.Cuts"))
 (gr_line (start 187.5 110.5) (end 187.5 97.5) (stroke (width 0.05) (type default)) (layer "Edge.Cuts"))
 (gr_line (start 190.5 55.5) (end 190.5 61.5) (stroke (width 0.05) (type default)) (layer "Edge.Cuts"))
 (gr_line (start 190.5 61.5) (end 204 61.5) (stroke (width 0.05) (type default)) (layer "Edge.Cuts"))
 (gr_line (start 204 61.5) (end 204 72) (stroke (width 0.05) (type default)) (layer "Edge.Cuts"))
 (gr_line (start 204 72) (end 187 72) (stroke (width 0.05) (type default)) (layer "Edge.Cuts"))
 (segment (start 144.836 78.985) (end 144.836 80.719314) (width 0.2) (layer "F.Cu") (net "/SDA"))
 (segment (start 135.335315 94.43) (end 142.845315 86.92) (width 0.2) (layer "F.Cu") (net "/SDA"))
 (segment (start 124.486598 94.43) (end 135.335315 94.43) (width 0.2) (layer "F.Cu") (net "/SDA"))
 (segment (start 153.609 70.212) (end 144.836 78.985) (width 0.2) (layer "F.Cu") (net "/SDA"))
 (segment (start 120.25 90.193402) (end 124.486598 94.43) (width 0.2) (layer "F.Cu") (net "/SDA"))
 (segment (start 159.715 70.212) (end 153.609 70.212) (width 0.2) (layer "F.Cu") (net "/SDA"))
 (segment (start 136.595213 88.960101) (end 123.05 88.960101) (width 0.2) (layer "F.Cu") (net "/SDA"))
 (segment (start 121.070101 88.14) (end 120.25 88.960101) (width 0.2) (layer "F.Cu") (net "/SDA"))
 (segment (start 123.05 88.960101) (end 122.229899 88.14) (width 0.2) (layer "F.Cu") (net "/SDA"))
 (segment (start 144.836 80.719314) (end 136.595213 88.960101) (width 0.2) (layer "F.Cu") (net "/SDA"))
 (segment (start 142.845315 86.92) (end 160 86.92) (width 0.2) (layer "F.Cu") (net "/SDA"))
 (segment (start 120.25 88.960101) (end 120.25 90.193402) (width 0.2) (layer "F.Cu") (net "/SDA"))
 (segment (start 122.229899 88.14) (end 121.070101 88.14) (width 0.2) (layer "F.Cu") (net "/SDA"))
 (segment (start 145.151 86.92) (end 160 86.92) (width 0.2) (layer "B.Cu") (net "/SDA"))
 (segment (start 138.366 80.135) (end 145.151 86.92) (width 0.2) (layer "B.Cu") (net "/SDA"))
 (segment (start 145.5 49) (end 146.5 50) (width 0.2) (layer "F.Cu") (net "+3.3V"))
 (segment (start 160 78.472) (end 160 79.3) (width 0.2) (layer "F.Cu") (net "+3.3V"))
 (segment (start 175.88 62.592) (end 160 78.472) (width 0.2) (layer "F.Cu") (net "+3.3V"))
 (segment (start 145.5 44.5) (end 145.5 49) (width 0.2) (layer "F.Cu") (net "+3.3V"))
 (segment (start 146.5 77.081) (end 143.446 80.135) (width 0.2) (layer "B.Cu") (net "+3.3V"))
 (segment (start 143.446 80.135) (end 146.301 82.99) (width 0.2) (layer "B.Cu") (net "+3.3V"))
 (segment (start 146.5 50) (end 146.5 77.081) (width 0.2) (layer "B.Cu") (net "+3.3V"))
 (segment (start 146.301 82.99) (end 156.31 82.99) (width 0.2) (layer "B.Cu") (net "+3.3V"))
 (segment (start 156.31 82.99) (end 160 79.3) (width 0.2) (layer "B.Cu") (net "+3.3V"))
 (segment (start 158.85 76.130642) (end 167.89 67.090642) (width 0.2) (layer "F.Cu") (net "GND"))
 (segment (start 167.89 60.19) (end 169.04 59.04) (width 0.2) (layer "F.Cu") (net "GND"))
 (segment (start 121.65 89.54) (end 136.581 89.54) (width 0.2) (layer "F.Cu") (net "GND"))
 (segment (start 160 81.84) (end 158.85 80.69) (width 0.2) (layer "F.Cu") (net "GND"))
 (segment (start 147.691 81.84) (end 160 81.84) (width 0.2) (layer "F.Cu") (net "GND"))
 (segment (start 167.89 67.090642) (end 167.89 60.19) (width 0.2) (layer "F.Cu") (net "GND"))
 (segment (start 169.04 59.04) (end 174.868 59.04) (width 0.2) (layer "F.Cu") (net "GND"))
 (segment (start 158.85 80.69) (end 158.85 76.130642) (width 0.2) (layer "F.Cu") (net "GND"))
 (segment (start 145.986 80.135) (end 147.691 81.84) (width 0.2) (layer "F.Cu") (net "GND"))
 (segment (start 136.581 89.54) (end 145.986 80.135) (width 0.2) (layer "F.Cu") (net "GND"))
 (segment (start 174.868 59.04) (end 175.88 60.052) (width 0.2) (layer "F.Cu") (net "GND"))
 (segment (start 128.61 50) (end 138.88 50) (width 0.2) (layer "B.Cu") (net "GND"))
 (segment (start 113.65 64.96) (end 128.61 50) (width 0.2) (layer "B.Cu") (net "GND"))
 (segment (start 113.65 81.54) (end 113.65 64.96) (width 0.2) (layer "B.Cu") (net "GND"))
 (segment (start 121.65 89.54) (end 113.65 81.54) (width 0.2) (layer "B.Cu") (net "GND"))
 (segment (start 165.35 66.279044) (end 165.35 61.103654) (width 0.2) (layer "F.Cu") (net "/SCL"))
 (segment (start 166.023654 60.43) (end 166.976346 60.43) (width 0.2) (layer "F.Cu") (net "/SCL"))
 (segment (start 168.563654 57.89) (end 172.988358 57.89) (width 0.2) (layer "F.Cu") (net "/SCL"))
 (segment (start 177.093642 56.212) (end 177.555 56.673358) (width 0.2) (layer "F.Cu") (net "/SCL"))
 (segment (start 167.89 58.563654) (end 168.563654 57.89) (width 0.2) (layer "F.Cu") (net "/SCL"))
 (segment (start 163.957044 67.672) (end 165.35 66.279044) (width 0.2) (layer "F.Cu") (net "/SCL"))
 (segment (start 174.666358 56.212) (end 177.093642 56.212) (width 0.2) (layer "F.Cu") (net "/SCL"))
 (segment (start 172.988358 57.89) (end 174.666358 56.212) (width 0.2) (layer "F.Cu") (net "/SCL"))
 (segment (start 166.976346 60.43) (end 167.89 59.516346) (width 0.2) (layer "F.Cu") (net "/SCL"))
 (segment (start 177.555 56.673358) (end 177.555 73.590642) (width 0.2) (layer "F.Cu") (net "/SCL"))
 (segment (start 177.555 73.590642) (end 166.765642 84.38) (width 0.2) (layer "F.Cu") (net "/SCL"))
 (segment (start 165.35 61.103654) (end 166.023654 60.43) (width 0.2) (layer "F.Cu") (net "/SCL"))
 (segment (start 166.765642 84.38) (end 160 84.38) (width 0.2) (layer "F.Cu") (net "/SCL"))
 (segment (start 159.715 67.672) (end 163.957044 67.672) (width 0.2) (layer "F.Cu") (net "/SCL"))
 (segment (start 167.89 59.516346) (end 167.89 58.563654) (width 0.2) (layer "F.Cu") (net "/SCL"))
 (segment (start 160 84.38) (end 145.151 84.38) (width 0.2) (layer "B.Cu") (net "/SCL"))
 (segment (start 145.151 84.38) (end 140.906 80.135) (width 0.2) (layer "B.Cu") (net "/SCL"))
 (segment (start 143.96 51.06066) (end 152.95134 60.052) (width 0.2) (layer "F.Cu") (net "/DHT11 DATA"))
 (segment (start 143.96 50) (end 143.96 51.06066) (width 0.2) (layer "F.Cu") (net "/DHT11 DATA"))
 (segment (start 152.95134 60.052) (end 159.715 60.052) (width 0.2) (layer "F.Cu") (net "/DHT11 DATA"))
 (segment (start 143.38 50) (end 143.96 50) (width 0.2) (layer "F.Cu") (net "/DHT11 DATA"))
 (segment (start 137.88 44.5) (end 143.38 50) (width 0.2) (layer "F.Cu") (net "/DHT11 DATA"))
 (segment (start 159.543 62.42) (end 159.715 62.592) (width 0.2) (layer "F.Cu") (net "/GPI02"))
 (segment (start 120 62.42) (end 159.543 62.42) (width 0.2) (layer "F.Cu") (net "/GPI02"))
 (segment (start 149.868 65.132) (end 128 87) (width 0.2) (layer "F.Cu") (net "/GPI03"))
 (segment (start 159.715 65.132) (end 149.868 65.132) (width 0.2) (layer "F.Cu") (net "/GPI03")))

